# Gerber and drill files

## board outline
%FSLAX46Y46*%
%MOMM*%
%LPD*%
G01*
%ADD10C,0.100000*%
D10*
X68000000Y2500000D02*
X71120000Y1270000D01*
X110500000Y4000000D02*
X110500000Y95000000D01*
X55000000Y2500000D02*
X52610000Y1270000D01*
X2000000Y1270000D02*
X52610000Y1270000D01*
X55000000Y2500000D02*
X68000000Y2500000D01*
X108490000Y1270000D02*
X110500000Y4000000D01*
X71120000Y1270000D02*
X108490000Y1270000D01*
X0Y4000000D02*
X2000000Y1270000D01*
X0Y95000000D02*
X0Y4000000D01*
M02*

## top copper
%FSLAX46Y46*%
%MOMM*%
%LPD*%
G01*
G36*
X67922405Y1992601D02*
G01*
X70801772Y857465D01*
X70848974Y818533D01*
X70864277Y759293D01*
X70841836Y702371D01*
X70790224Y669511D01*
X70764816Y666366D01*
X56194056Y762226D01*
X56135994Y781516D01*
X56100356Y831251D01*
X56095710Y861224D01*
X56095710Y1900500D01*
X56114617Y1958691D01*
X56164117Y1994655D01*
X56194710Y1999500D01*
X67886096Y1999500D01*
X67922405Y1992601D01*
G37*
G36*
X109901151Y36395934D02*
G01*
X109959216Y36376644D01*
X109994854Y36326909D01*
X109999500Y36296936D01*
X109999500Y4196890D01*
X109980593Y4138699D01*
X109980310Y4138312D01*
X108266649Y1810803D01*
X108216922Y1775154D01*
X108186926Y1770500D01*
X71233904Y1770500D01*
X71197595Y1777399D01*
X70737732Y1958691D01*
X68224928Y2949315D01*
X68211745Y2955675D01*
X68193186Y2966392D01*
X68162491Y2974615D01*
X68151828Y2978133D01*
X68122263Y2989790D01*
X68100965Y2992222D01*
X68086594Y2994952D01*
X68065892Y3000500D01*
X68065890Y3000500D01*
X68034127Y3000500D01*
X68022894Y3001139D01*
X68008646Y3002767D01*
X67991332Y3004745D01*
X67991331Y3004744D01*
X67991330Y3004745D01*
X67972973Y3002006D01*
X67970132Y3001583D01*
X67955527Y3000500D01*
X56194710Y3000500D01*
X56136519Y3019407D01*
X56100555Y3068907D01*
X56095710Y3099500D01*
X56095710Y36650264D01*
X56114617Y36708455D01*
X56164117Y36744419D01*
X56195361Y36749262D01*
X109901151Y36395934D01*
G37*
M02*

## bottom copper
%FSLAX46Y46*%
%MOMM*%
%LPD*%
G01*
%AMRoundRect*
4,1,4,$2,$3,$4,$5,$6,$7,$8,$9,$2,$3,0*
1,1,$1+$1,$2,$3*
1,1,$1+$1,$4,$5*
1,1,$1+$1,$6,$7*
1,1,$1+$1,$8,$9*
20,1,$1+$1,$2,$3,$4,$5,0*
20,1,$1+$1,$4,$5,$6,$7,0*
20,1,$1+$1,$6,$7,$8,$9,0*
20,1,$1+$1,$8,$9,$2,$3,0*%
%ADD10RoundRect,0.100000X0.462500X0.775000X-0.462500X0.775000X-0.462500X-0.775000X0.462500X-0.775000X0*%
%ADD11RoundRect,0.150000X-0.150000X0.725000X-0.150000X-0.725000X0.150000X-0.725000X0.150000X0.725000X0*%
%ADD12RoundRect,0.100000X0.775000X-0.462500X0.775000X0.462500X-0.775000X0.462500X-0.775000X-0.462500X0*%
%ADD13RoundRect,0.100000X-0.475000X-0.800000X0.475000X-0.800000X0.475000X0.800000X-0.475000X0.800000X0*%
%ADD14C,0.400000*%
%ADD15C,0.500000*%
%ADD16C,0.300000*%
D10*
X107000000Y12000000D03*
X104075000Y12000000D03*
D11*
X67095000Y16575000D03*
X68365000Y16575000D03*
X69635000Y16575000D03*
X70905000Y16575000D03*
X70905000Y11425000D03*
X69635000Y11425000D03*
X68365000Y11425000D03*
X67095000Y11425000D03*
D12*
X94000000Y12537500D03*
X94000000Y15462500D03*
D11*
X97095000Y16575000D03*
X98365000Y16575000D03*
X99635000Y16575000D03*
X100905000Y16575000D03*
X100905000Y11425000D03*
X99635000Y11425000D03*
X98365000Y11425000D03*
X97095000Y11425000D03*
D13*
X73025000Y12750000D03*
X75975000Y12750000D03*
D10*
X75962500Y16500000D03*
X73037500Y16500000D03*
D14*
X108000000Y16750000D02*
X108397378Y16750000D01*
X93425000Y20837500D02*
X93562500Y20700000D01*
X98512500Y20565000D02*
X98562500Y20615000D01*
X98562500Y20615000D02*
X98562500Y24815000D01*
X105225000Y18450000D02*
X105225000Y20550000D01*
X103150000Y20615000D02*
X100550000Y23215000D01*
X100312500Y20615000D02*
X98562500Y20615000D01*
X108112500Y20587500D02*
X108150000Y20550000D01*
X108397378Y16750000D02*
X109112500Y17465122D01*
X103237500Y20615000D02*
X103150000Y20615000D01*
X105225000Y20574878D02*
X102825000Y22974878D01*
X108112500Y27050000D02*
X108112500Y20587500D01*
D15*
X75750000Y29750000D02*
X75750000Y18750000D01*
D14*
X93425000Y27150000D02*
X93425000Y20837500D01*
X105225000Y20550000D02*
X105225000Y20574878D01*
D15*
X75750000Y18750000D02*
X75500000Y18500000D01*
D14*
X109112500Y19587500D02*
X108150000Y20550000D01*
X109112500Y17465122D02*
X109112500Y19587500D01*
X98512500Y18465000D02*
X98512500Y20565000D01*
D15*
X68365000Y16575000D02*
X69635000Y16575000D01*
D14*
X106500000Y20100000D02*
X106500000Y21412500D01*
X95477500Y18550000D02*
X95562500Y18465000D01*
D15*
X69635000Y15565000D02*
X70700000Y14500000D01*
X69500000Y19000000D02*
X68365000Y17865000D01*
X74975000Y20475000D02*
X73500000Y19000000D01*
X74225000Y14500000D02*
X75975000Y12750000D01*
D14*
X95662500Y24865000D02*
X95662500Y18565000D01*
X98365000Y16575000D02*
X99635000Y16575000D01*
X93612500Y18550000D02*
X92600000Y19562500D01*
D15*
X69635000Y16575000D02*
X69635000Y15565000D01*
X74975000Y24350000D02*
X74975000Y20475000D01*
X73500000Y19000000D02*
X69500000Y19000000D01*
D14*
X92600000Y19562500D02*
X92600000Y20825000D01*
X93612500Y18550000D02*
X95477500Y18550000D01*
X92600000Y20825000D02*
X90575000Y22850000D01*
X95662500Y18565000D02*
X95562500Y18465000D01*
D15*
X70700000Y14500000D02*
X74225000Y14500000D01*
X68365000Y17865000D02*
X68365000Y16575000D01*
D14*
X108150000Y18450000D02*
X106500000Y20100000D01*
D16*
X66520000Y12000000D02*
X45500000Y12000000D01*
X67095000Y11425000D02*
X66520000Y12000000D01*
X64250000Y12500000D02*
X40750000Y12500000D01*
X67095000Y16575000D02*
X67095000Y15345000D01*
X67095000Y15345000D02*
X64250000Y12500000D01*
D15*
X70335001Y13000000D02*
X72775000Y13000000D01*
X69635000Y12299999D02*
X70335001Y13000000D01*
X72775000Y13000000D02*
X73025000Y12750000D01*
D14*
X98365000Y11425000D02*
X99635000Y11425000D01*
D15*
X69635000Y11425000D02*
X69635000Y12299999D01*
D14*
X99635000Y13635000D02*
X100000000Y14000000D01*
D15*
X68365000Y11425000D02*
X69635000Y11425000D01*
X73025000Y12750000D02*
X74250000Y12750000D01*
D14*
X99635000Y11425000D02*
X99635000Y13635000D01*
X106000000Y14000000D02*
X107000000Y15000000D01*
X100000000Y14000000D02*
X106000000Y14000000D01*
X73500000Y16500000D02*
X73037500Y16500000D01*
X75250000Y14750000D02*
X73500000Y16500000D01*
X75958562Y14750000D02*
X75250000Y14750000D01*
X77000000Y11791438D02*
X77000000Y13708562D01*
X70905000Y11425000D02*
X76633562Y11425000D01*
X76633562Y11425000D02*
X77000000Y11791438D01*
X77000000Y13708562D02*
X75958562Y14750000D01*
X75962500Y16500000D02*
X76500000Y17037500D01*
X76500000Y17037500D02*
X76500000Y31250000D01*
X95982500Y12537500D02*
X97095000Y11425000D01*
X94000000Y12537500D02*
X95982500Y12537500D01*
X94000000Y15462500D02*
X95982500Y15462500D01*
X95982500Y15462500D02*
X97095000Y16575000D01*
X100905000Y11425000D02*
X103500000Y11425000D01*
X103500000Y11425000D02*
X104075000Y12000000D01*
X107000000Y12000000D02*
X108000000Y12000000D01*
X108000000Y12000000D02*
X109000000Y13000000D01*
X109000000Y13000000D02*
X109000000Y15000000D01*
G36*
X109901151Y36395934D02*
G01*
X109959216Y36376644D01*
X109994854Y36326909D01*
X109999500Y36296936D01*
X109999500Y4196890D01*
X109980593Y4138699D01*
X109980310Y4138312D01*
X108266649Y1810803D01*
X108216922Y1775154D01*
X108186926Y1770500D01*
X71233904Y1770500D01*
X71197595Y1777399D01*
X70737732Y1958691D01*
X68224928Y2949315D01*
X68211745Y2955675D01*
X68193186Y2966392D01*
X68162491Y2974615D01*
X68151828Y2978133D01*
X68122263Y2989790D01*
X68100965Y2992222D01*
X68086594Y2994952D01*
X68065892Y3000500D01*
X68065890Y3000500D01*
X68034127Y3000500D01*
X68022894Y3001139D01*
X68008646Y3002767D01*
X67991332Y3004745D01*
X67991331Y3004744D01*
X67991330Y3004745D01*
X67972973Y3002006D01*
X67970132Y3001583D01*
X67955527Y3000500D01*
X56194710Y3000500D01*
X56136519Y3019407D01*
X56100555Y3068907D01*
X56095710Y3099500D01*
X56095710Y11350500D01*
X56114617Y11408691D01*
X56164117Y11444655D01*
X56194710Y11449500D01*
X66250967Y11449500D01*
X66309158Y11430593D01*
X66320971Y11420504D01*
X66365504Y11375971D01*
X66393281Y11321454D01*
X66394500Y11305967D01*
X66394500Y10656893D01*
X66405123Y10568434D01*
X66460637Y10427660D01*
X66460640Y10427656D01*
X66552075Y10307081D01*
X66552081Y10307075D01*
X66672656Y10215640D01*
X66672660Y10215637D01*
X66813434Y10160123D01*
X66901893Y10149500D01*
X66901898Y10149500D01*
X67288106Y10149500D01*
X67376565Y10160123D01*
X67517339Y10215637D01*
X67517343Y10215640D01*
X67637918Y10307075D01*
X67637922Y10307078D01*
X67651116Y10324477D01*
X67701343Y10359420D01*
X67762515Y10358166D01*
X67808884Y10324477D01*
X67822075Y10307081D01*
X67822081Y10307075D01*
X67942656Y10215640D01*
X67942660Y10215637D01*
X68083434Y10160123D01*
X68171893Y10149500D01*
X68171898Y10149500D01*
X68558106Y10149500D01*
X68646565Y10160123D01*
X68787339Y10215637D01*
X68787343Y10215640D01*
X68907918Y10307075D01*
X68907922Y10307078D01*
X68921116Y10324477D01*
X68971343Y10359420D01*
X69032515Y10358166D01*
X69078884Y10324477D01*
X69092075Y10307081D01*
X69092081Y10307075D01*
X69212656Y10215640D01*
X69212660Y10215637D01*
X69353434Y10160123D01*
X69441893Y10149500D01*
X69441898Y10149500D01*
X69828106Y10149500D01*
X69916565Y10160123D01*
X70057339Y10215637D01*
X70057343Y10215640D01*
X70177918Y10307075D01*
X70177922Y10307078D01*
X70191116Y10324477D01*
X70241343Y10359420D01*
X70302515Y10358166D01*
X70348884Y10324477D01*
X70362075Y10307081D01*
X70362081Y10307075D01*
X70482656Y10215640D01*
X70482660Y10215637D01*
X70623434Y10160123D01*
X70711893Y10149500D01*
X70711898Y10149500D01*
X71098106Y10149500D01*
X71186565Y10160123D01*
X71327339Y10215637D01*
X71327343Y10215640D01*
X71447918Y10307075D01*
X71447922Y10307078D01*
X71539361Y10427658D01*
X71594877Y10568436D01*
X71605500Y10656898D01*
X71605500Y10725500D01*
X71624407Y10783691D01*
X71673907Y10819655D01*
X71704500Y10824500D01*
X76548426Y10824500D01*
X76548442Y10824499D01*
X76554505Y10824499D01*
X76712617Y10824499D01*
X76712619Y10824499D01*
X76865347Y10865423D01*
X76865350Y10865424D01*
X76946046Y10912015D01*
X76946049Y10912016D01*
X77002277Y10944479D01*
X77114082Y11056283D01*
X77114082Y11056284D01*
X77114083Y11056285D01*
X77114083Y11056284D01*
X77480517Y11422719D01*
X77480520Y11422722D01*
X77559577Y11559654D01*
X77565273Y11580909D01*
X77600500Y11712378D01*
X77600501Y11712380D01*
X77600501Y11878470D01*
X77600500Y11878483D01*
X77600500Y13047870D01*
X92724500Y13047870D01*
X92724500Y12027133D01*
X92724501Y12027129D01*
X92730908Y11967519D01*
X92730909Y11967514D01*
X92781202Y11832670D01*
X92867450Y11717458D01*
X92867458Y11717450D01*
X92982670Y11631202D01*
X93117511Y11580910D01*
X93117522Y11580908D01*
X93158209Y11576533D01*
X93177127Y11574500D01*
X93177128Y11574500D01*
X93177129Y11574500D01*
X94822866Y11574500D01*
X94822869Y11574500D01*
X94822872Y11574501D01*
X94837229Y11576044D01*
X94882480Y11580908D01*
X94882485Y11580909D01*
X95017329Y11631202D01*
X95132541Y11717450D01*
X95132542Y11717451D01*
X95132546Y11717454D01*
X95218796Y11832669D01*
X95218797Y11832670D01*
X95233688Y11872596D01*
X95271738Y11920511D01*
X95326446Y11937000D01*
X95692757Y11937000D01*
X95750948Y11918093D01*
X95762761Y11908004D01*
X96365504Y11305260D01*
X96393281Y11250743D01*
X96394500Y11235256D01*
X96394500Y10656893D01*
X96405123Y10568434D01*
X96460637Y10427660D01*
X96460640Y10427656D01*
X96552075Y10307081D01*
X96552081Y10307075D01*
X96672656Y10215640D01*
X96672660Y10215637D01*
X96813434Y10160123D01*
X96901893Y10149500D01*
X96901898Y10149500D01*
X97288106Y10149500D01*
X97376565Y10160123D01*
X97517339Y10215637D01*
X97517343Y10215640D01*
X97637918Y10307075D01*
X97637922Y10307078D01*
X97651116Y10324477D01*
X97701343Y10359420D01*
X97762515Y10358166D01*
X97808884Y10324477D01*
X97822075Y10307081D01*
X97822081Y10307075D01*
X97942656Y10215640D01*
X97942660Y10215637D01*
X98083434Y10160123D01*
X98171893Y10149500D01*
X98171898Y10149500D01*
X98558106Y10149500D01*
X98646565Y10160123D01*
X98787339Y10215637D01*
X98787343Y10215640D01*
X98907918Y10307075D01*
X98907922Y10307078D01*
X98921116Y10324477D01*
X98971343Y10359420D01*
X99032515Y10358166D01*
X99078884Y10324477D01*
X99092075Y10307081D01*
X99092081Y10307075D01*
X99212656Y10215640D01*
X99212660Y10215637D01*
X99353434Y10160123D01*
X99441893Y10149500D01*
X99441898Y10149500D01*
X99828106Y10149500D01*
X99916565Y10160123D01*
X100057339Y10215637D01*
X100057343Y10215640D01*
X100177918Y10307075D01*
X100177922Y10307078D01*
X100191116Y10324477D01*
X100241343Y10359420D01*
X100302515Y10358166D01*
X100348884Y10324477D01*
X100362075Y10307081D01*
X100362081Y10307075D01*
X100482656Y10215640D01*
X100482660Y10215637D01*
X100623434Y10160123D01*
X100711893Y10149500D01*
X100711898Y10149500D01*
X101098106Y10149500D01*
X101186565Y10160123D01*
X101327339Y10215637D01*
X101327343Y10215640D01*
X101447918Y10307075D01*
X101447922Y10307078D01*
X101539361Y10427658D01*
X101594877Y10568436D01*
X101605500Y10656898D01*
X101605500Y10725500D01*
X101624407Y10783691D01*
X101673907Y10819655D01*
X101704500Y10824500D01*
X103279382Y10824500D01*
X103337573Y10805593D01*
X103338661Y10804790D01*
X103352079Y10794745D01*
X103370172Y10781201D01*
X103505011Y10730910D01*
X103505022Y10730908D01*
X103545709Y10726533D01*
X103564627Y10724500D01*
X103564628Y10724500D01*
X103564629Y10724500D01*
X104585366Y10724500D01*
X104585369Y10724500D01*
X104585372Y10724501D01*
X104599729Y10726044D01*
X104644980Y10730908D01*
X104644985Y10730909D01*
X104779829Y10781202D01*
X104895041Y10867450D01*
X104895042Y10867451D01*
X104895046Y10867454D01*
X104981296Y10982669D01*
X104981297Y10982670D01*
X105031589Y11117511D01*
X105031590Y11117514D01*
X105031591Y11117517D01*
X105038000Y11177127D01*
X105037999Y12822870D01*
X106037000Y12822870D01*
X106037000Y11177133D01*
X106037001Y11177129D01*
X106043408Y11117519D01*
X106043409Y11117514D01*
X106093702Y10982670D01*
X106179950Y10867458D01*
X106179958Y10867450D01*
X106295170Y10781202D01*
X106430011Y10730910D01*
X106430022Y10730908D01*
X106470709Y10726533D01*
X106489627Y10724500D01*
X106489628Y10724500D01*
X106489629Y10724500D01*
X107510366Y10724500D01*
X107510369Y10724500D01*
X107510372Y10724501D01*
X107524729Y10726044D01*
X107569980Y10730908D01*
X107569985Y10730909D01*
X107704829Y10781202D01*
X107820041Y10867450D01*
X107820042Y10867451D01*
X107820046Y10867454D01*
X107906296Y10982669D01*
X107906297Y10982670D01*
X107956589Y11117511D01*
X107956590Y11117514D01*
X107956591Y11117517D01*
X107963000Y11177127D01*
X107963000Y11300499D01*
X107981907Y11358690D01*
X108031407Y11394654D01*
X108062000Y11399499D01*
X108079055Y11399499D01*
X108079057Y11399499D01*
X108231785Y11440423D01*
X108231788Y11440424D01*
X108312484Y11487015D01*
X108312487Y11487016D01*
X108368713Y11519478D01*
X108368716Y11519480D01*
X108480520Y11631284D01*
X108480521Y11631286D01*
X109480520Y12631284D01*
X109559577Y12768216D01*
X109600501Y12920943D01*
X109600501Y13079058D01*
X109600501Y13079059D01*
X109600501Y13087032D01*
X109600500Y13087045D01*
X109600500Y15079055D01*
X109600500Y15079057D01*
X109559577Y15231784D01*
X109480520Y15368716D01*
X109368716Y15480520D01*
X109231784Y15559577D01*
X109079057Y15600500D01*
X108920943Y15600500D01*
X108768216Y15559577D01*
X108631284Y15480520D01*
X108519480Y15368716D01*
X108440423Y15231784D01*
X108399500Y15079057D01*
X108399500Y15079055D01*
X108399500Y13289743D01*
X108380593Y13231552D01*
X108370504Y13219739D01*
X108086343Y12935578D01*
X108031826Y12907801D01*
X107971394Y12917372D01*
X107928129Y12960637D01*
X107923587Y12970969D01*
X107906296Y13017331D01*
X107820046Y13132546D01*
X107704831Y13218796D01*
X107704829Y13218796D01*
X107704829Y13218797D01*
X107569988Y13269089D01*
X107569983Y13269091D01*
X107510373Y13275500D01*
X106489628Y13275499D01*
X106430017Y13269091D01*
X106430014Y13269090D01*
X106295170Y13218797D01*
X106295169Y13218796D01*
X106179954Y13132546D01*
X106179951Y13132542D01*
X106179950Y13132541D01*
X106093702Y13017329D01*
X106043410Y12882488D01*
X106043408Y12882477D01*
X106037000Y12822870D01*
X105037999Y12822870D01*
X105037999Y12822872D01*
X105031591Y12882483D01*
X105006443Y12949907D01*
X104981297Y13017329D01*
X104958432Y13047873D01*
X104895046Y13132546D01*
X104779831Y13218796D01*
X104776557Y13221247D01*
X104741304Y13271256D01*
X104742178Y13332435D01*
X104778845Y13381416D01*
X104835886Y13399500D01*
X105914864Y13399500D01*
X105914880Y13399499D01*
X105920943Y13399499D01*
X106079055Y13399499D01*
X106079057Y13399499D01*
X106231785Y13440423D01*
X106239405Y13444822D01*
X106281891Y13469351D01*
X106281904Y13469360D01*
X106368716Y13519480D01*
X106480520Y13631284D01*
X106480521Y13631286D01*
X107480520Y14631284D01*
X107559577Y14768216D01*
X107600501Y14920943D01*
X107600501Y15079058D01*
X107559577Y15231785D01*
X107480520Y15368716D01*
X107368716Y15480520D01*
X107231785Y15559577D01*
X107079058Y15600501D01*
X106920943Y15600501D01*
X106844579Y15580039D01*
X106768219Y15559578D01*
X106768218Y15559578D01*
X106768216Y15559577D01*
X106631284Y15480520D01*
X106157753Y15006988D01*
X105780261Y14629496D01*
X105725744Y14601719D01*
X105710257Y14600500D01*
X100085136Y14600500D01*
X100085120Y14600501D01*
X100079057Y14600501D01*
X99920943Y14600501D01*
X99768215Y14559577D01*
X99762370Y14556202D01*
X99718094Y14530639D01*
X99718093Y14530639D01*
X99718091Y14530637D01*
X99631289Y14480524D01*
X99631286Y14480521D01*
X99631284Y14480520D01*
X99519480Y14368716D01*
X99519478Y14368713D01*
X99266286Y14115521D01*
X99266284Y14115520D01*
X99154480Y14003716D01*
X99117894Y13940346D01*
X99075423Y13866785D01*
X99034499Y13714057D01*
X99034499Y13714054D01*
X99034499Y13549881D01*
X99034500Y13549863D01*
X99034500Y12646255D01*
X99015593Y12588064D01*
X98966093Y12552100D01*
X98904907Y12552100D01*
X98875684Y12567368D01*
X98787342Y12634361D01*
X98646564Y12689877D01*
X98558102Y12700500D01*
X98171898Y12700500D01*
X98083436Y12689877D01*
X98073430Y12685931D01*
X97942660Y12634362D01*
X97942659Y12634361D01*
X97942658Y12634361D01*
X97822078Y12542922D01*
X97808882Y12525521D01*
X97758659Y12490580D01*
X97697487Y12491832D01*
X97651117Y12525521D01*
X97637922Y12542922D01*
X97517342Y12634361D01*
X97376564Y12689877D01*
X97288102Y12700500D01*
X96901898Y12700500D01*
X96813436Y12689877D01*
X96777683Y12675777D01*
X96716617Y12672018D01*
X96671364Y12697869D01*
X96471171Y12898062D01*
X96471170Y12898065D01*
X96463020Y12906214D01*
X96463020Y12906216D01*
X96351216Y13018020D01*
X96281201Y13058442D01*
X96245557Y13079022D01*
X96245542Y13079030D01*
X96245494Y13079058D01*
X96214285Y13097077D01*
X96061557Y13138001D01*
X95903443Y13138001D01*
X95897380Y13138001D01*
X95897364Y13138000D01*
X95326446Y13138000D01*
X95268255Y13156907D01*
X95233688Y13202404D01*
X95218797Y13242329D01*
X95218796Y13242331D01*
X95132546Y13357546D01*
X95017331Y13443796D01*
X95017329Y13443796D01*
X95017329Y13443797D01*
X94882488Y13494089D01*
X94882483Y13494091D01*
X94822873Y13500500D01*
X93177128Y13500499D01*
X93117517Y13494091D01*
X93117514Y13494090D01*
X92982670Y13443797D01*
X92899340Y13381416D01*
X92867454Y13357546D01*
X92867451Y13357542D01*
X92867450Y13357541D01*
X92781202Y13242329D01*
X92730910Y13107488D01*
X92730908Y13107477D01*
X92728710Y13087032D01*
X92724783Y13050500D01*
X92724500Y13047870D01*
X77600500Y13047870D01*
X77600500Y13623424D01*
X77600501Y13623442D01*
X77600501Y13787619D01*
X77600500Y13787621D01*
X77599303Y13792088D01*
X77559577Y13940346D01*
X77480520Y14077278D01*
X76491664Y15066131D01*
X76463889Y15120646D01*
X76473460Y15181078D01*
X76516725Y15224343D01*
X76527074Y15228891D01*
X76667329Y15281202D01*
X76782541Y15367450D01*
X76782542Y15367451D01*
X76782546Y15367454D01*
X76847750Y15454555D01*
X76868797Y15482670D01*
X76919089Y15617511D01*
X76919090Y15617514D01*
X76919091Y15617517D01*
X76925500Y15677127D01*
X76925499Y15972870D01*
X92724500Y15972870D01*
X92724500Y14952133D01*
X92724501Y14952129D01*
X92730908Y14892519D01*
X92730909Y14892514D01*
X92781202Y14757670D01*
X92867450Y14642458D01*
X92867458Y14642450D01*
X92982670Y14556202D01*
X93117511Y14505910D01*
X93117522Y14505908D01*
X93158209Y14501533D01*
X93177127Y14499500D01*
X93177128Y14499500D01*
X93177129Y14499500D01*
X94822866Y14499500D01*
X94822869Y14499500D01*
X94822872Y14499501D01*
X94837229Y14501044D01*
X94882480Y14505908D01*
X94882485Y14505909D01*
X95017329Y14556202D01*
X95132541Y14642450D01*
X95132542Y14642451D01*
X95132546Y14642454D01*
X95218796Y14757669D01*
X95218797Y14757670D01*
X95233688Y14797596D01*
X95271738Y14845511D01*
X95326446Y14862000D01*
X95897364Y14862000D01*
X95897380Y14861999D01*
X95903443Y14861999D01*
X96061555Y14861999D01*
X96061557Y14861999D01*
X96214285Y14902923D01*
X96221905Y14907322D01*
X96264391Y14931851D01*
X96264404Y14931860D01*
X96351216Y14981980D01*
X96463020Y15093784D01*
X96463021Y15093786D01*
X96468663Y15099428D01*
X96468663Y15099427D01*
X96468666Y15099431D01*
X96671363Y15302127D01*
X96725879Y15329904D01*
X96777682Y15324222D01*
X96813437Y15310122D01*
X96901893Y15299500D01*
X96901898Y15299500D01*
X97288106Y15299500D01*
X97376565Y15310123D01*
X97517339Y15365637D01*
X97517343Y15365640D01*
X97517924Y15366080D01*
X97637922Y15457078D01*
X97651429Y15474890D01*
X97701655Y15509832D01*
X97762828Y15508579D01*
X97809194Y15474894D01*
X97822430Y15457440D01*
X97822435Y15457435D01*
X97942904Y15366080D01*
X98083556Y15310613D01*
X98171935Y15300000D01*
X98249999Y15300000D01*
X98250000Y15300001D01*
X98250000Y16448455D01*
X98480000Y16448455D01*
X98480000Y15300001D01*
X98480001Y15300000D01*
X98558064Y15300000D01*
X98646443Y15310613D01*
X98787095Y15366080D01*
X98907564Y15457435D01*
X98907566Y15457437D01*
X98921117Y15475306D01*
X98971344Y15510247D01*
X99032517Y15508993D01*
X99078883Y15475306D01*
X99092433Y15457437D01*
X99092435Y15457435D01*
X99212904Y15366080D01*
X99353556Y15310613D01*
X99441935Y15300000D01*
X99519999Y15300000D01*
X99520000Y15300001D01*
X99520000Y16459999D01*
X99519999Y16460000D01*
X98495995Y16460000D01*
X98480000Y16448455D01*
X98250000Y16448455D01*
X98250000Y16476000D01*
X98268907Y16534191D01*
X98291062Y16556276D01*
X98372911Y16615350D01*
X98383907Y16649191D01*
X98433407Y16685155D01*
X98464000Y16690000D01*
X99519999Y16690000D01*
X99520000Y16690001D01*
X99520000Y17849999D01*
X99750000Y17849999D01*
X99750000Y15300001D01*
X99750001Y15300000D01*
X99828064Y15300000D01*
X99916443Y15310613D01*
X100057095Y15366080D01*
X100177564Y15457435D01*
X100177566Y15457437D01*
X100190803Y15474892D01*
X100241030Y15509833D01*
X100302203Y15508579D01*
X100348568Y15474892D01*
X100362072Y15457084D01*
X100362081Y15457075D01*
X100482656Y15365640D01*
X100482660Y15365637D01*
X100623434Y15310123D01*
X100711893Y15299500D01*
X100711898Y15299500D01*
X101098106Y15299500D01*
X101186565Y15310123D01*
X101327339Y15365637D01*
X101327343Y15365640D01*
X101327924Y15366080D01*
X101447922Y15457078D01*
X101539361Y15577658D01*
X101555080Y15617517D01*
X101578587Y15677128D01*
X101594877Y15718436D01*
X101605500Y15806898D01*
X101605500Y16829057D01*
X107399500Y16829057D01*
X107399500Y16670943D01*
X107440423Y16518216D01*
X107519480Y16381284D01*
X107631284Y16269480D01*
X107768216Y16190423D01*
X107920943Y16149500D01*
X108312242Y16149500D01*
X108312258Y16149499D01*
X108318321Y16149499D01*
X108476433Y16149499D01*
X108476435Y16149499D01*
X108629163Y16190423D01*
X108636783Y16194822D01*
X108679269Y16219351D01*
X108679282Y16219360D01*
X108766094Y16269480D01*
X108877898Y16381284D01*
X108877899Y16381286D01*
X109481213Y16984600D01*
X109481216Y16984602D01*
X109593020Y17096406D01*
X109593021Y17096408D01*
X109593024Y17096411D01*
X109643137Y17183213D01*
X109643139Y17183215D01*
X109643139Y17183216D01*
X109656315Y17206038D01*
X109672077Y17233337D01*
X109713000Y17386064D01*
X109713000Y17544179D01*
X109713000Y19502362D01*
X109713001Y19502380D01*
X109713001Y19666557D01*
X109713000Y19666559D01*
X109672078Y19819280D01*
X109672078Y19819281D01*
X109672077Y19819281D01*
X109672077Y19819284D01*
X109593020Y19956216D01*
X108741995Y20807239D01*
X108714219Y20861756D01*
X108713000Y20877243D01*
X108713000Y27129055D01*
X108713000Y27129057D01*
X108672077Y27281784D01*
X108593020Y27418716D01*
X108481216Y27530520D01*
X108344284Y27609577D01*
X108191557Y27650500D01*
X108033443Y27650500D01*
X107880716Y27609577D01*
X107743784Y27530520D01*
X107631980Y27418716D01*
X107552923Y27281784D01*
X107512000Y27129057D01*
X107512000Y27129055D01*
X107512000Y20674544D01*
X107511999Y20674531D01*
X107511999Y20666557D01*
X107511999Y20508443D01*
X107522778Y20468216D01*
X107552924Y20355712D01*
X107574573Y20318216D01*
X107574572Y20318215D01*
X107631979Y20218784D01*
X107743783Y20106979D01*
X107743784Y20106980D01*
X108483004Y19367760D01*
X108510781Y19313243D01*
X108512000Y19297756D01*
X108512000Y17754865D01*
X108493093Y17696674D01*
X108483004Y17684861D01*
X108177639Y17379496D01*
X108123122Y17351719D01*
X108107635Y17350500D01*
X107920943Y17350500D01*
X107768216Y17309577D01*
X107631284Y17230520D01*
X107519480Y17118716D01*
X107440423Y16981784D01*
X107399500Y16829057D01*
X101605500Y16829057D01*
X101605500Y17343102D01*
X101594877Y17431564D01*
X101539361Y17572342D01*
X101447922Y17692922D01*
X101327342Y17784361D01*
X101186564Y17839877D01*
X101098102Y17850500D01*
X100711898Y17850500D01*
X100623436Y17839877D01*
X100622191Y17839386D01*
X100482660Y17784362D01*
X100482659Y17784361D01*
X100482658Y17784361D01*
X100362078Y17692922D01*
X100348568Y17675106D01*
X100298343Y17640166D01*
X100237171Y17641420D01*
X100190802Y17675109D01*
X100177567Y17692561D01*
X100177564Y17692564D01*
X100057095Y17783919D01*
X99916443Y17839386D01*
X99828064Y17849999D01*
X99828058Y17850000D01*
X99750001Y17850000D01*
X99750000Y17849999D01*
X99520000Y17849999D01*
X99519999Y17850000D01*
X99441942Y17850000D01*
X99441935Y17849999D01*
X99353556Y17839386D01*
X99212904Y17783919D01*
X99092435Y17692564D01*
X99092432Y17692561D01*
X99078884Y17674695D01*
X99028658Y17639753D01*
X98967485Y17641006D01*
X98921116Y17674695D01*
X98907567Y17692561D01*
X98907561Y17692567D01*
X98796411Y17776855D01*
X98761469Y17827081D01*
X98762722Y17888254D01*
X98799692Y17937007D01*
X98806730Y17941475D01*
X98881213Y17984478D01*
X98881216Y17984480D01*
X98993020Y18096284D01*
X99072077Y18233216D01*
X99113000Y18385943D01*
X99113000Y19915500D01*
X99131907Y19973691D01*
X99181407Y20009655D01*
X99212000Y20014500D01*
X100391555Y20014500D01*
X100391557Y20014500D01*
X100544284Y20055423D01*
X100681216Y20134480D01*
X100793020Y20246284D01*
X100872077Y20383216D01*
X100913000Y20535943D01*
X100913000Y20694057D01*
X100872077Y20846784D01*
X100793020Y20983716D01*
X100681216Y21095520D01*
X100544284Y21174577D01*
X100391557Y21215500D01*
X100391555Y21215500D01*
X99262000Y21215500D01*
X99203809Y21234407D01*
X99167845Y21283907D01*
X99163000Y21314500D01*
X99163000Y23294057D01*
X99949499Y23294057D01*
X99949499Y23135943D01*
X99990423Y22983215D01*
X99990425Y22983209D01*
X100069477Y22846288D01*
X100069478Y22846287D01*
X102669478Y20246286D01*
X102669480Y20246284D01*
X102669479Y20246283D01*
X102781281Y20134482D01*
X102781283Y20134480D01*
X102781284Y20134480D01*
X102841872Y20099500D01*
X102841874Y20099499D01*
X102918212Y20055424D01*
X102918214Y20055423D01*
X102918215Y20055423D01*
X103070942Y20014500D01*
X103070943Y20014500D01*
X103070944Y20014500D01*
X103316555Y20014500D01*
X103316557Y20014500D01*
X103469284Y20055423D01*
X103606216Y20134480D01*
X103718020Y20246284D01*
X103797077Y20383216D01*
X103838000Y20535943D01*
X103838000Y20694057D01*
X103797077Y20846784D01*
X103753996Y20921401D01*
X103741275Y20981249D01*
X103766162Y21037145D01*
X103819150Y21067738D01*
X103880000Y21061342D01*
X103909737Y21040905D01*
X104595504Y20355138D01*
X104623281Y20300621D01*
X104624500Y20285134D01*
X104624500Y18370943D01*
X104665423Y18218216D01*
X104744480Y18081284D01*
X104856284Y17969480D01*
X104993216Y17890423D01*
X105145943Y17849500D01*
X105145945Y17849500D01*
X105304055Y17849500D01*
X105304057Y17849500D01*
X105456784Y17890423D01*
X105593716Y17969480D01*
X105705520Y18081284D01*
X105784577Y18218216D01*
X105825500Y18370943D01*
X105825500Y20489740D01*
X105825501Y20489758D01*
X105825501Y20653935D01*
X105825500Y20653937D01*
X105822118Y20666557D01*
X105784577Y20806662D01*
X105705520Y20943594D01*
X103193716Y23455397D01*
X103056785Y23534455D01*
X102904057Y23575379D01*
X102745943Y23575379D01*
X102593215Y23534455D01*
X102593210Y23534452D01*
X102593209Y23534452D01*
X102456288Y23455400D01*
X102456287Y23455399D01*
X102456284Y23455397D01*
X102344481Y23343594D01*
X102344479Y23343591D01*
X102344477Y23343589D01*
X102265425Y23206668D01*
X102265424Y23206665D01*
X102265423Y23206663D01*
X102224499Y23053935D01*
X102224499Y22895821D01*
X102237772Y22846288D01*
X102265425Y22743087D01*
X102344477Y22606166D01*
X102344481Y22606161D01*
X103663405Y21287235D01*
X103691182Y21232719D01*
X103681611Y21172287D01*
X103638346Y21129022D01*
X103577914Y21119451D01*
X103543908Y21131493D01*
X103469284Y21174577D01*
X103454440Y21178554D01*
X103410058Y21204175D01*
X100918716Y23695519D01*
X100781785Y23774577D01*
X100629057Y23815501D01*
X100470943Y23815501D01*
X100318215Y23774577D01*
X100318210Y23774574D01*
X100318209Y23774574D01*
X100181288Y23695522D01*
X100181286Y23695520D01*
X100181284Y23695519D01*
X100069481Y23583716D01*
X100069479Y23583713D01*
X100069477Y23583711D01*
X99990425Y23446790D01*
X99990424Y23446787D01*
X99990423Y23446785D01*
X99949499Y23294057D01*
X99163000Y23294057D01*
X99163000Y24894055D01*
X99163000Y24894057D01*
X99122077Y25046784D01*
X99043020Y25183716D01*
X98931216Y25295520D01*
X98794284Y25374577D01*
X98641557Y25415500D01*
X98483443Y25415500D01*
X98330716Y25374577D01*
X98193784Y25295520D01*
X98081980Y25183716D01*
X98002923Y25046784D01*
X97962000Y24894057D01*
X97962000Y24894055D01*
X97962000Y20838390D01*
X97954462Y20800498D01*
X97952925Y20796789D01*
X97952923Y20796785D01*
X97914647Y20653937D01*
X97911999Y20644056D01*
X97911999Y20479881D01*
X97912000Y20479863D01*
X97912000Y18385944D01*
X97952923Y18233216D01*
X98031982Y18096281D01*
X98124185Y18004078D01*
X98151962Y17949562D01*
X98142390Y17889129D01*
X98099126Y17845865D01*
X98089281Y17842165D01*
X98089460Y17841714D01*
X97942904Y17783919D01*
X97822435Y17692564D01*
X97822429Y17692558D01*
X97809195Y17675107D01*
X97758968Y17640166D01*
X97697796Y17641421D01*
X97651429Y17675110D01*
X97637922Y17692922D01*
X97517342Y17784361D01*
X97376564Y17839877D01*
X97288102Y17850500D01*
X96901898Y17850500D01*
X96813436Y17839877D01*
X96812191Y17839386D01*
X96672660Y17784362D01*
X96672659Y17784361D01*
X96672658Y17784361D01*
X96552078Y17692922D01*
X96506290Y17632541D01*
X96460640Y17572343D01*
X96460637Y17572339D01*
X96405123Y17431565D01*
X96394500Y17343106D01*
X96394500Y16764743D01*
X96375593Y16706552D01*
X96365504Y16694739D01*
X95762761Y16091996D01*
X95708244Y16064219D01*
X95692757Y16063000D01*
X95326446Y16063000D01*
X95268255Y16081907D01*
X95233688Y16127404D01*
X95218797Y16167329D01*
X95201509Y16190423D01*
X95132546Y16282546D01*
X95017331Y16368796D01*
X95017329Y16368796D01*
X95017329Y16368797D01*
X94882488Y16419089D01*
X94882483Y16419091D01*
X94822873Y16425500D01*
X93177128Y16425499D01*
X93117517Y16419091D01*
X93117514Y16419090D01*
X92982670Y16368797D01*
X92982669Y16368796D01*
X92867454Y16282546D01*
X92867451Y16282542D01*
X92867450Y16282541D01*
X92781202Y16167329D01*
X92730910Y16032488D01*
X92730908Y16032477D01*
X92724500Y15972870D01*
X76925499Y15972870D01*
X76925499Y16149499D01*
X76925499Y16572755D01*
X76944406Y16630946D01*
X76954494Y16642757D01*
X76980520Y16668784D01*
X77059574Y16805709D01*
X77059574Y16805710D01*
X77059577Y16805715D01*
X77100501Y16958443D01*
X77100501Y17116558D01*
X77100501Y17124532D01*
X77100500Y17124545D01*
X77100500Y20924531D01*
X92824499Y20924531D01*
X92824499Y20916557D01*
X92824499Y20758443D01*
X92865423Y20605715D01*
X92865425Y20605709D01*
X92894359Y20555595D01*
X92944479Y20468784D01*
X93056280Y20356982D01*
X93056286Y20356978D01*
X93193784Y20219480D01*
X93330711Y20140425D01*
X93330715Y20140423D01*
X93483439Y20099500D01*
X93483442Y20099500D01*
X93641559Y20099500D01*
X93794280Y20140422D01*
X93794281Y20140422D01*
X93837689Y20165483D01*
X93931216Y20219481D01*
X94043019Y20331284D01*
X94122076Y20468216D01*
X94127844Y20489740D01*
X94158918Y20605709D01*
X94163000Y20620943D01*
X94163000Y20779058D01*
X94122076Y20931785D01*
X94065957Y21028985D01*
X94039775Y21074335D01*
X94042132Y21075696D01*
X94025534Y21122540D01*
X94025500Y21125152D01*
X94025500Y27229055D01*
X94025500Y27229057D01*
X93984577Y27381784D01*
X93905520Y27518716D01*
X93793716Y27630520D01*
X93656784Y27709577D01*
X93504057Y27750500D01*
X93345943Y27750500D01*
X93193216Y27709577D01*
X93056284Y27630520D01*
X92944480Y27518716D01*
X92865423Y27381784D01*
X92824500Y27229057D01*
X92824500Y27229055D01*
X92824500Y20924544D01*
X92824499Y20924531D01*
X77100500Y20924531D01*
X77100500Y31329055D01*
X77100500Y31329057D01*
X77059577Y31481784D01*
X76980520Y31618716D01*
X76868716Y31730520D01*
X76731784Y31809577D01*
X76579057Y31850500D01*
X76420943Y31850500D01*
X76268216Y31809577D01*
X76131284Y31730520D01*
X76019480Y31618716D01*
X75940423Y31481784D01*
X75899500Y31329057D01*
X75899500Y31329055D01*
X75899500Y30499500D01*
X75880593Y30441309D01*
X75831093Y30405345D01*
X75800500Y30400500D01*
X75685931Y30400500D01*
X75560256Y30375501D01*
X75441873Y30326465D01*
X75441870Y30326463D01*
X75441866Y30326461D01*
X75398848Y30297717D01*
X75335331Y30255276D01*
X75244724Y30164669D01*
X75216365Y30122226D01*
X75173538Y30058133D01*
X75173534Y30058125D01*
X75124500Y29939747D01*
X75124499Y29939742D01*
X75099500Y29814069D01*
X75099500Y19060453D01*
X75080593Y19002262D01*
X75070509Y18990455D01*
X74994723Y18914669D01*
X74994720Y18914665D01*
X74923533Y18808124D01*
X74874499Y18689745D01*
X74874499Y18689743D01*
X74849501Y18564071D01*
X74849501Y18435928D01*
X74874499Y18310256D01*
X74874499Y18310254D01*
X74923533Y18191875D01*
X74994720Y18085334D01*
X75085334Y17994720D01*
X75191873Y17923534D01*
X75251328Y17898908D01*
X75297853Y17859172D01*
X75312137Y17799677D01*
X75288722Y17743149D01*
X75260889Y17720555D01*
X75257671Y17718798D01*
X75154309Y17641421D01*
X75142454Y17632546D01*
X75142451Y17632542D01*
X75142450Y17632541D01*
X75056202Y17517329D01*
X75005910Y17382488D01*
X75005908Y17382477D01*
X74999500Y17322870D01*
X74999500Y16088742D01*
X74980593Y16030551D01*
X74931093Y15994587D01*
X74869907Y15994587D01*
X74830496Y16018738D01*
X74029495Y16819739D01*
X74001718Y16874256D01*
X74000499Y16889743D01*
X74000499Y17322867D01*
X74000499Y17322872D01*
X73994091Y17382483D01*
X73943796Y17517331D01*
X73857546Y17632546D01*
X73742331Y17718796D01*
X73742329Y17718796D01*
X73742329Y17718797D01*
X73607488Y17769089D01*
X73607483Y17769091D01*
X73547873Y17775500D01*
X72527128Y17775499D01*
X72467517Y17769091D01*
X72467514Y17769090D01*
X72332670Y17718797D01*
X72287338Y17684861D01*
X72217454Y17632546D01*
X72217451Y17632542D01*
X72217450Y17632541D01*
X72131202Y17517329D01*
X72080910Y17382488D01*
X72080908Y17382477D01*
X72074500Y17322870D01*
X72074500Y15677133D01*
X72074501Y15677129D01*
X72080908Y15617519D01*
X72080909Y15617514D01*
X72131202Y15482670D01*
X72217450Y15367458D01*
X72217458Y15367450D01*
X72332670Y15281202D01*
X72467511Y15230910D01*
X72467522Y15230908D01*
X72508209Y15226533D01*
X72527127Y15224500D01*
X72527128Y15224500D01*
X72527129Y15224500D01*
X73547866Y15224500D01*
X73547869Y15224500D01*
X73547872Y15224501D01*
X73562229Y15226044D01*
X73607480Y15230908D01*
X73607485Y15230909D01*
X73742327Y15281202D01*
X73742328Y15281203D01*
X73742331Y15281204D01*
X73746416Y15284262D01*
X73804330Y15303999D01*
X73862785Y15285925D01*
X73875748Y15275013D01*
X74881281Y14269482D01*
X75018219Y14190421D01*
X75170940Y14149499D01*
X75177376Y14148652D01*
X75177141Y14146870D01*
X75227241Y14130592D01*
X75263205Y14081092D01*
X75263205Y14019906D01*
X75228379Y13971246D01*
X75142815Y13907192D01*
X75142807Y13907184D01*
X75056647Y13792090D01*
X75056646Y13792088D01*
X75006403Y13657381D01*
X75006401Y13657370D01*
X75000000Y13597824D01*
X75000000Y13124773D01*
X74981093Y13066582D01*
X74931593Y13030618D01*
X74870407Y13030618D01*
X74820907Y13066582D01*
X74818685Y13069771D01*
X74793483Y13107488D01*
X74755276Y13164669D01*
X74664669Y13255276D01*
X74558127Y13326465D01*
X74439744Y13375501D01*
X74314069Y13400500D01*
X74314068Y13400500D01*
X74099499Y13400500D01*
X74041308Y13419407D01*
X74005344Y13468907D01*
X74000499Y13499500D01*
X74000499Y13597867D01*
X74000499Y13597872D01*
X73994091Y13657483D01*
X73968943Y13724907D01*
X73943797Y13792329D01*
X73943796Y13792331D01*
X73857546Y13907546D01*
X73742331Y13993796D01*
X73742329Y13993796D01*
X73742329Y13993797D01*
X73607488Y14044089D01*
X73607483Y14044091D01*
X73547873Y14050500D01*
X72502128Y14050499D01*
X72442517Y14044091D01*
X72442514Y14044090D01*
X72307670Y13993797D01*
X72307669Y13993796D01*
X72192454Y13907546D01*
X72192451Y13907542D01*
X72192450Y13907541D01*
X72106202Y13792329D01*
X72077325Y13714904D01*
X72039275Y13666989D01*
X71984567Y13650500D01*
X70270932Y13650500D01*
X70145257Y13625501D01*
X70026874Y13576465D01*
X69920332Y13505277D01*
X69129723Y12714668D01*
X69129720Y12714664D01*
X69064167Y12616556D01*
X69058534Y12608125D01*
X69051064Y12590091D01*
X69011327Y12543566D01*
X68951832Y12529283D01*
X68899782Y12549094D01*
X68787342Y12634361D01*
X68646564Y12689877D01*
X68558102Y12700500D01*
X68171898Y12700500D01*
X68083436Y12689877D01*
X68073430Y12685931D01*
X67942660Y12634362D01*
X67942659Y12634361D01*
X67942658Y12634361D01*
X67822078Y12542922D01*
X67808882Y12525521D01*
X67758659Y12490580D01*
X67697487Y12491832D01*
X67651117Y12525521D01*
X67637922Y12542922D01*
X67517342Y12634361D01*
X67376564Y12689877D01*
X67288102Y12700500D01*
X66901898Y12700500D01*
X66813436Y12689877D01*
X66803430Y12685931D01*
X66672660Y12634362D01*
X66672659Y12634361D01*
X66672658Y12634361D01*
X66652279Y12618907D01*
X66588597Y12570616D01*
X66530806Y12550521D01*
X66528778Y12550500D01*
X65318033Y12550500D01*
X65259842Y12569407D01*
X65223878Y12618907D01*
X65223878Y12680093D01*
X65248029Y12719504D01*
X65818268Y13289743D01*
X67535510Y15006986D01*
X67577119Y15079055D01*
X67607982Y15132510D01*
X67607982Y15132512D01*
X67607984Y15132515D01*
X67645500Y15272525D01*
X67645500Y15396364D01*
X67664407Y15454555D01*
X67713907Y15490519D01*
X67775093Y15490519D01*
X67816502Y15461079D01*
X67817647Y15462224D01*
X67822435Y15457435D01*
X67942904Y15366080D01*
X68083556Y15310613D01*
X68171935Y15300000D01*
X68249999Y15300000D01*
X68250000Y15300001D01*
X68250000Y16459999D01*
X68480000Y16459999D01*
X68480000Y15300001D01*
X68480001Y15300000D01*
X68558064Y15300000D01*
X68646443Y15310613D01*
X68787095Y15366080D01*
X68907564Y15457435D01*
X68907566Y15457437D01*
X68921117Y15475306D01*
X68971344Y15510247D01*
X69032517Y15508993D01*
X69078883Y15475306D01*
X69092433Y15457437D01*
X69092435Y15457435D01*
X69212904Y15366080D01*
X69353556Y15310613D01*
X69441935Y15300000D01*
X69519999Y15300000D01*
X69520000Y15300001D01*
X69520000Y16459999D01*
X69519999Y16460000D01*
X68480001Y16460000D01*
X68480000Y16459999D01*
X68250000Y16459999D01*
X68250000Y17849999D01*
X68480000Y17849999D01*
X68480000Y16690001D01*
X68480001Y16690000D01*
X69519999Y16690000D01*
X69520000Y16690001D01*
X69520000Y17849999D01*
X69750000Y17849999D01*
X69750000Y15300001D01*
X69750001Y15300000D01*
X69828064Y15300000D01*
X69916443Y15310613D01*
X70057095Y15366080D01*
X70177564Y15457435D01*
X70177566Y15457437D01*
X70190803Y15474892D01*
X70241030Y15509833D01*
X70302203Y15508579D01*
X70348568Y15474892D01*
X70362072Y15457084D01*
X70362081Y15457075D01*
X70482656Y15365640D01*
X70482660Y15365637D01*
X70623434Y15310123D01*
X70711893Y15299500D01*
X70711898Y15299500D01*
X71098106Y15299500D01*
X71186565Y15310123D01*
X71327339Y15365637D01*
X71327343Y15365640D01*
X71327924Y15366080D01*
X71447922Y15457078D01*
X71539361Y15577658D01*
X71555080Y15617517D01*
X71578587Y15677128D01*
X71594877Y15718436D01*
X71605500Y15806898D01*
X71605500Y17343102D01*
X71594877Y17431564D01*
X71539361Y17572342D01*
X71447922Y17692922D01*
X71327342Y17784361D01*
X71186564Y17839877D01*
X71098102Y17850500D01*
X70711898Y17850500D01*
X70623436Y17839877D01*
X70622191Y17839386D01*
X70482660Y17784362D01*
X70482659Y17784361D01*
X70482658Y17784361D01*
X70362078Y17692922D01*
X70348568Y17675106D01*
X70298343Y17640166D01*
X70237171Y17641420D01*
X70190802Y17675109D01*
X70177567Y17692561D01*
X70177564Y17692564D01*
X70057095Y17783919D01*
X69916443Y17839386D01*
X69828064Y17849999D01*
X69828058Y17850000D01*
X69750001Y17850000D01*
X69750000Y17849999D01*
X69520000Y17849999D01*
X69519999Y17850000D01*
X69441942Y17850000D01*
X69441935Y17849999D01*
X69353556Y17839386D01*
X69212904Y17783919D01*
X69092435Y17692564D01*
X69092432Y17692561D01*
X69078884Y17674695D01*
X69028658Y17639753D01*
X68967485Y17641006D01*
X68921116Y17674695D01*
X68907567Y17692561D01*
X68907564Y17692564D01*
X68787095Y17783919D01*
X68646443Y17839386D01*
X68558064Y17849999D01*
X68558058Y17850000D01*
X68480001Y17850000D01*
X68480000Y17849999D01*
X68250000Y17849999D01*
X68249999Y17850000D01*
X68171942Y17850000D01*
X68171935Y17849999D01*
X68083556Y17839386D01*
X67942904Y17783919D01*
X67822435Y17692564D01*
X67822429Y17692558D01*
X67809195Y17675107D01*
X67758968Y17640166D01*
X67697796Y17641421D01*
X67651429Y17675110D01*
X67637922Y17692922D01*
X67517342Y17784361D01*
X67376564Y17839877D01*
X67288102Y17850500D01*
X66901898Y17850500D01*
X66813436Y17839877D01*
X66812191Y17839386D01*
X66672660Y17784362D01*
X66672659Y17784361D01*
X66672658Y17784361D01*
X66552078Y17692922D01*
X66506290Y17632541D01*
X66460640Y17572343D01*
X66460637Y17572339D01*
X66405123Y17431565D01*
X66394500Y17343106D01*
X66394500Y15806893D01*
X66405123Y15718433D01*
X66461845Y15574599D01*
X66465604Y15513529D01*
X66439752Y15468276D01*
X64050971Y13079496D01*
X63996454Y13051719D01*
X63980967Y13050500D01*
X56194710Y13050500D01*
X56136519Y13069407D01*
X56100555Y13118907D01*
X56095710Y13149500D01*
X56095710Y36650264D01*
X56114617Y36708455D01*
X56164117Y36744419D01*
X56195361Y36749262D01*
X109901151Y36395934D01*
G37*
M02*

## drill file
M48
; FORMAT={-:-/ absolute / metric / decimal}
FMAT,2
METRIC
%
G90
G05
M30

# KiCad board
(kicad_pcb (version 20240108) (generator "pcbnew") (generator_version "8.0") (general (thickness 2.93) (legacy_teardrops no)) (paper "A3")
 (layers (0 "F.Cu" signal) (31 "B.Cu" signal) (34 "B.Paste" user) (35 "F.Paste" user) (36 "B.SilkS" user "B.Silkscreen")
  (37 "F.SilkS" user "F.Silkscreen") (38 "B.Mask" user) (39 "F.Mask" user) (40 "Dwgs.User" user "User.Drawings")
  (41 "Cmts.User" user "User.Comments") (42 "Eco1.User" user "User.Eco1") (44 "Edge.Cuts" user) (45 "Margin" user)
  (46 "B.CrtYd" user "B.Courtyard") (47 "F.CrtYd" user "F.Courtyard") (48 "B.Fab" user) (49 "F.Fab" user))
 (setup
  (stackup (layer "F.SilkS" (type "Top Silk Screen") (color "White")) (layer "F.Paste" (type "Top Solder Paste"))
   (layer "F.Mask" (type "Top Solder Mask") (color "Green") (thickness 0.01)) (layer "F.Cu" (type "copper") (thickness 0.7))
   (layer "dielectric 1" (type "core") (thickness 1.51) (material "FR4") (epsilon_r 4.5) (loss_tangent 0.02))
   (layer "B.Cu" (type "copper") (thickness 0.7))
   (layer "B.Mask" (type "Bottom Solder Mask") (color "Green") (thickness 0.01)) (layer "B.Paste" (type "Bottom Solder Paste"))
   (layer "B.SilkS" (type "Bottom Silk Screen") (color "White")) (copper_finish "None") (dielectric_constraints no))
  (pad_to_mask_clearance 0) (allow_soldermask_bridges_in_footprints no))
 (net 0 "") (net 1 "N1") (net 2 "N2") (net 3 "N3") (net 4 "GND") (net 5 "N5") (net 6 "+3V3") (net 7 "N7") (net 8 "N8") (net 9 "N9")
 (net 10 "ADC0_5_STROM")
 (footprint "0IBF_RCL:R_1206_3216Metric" (layer "B.Cu") (at 105.5375 -12 180)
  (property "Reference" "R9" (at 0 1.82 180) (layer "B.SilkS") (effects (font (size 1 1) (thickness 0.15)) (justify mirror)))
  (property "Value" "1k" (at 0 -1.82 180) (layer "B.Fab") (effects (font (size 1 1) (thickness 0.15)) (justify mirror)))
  (pad "1" smd roundrect (at -1.4625 0 180) (size 1.125 1.75) (layers "B.Cu" "B.Paste" "B.Mask") (roundrect_rratio 0.08888888889)
   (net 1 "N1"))
  (pad "2" smd roundrect (at 1.4625 0 180) (size 1.125 1.75) (layers "B.Cu" "B.Paste" "B.Mask") (roundrect_rratio 0.08888888889)
   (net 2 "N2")))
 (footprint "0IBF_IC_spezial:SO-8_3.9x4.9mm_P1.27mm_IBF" (layer "B.Cu") (at 69 -14 -90)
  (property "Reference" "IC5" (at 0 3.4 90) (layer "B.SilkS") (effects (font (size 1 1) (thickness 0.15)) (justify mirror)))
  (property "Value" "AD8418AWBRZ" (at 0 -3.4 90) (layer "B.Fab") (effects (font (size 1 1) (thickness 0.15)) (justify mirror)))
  (pad "1" smd roundrect (at -2.575 1.905 270) (size 1.75 0.6) (layers "B.Cu" "B.Paste" "B.Mask") (roundrect_rratio 0.25) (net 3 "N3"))
  (pad "2" smd roundrect (at -2.575 0.635 270) (size 1.75 0.6) (layers "B.Cu" "B.Paste" "B.Mask") (roundrect_rratio 0.25) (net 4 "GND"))
  (pad "3" smd roundrect (at -2.575 -0.635 270) (size 1.75 0.6) (layers "B.Cu" "B.Paste" "B.Mask") (roundrect_rratio 0.25) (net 4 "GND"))
  (pad "4" smd roundrect (at -2.575 -1.905 270) (size 1.75 0.6) (layers "B.Cu" "B.Paste" "B.Mask") (roundrect_rratio 0.25))
  (pad "5" smd roundrect (at 2.575 -1.905 270) (size 1.75 0.6) (layers "B.Cu" "B.Paste" "B.Mask") (roundrect_rratio 0.25) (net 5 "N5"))
  (pad "6" smd roundrect (at 2.575 -0.635 270) (size 1.75 0.6) (layers "B.Cu" "B.Paste" "B.Mask") (roundrect_rratio 0.25) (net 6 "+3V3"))
  (pad "7" smd roundrect (at 2.575 0.635 270) (size 1.75 0.6) (layers "B.Cu" "B.Paste" "B.Mask") (roundrect_rratio 0.25) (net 6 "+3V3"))
  (pad "8" smd roundrect (at 2.575 1.905 270) (size 1.75 0.6) (layers "B.Cu" "B.Paste" "B.Mask") (roundrect_rratio 0.25) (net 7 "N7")))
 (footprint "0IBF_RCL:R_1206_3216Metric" (layer "B.Cu") (at 94 -14 90)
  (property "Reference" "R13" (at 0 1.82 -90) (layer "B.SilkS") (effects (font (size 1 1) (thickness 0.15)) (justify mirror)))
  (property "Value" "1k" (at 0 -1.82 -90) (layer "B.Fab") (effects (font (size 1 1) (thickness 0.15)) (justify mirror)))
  (pad "1" smd roundrect (at -1.4625 0 90) (size 1.125 1.75) (layers "B.Cu" "B.Paste" "B.Mask") (roundrect_rratio 0.08888888889)
   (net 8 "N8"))
  (pad "2" smd roundrect (at 1.4625 0 90) (size 1.125 1.75) (layers "B.Cu" "B.Paste" "B.Mask") (roundrect_rratio 0.08888888889) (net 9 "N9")))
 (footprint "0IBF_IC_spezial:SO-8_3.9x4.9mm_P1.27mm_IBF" (layer "B.Cu") (at 99 -14 -90)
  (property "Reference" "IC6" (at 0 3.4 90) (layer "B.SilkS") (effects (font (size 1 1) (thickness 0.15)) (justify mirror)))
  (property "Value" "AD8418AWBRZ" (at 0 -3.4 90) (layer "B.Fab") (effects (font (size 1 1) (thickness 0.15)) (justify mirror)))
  (pad "1" smd roundrect (at -2.575 1.905 270) (size 1.75 0.6) (layers "B.Cu" "B.Paste" "B.Mask") (roundrect_rratio 0.25) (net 9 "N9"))
  (pad "2" smd roundrect (at -2.575 0.635 270) (size 1.75 0.6) (layers "B.Cu" "B.Paste" "B.Mask") (roundrect_rratio 0.25) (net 4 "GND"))
  (pad "3" smd roundrect (at -2.575 -0.635 270) (size 1.75 0.6) (layers "B.Cu" "B.Paste" "B.Mask") (roundrect_rratio 0.25) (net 4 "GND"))
  (pad "4" smd roundrect (at -2.575 -1.905 270) (size 1.75 0.6) (layers "B.Cu" "B.Paste" "B.Mask") (roundrect_rratio 0.25))
  (pad "5" smd roundrect (at 2.575 -1.905 270) (size 1.75 0.6) (layers "B.Cu" "B.Paste" "B.Mask") (roundrect_rratio 0.25) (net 2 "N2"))
  (pad "6" smd roundrect (at 2.575 -0.635 270) (size 1.75 0.6) (layers "B.Cu" "B.Paste" "B.Mask") (roundrect_rratio 0.25) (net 6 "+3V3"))
  (pad "7" smd roundrect (at 2.575 0.635 270) (size 1.75 0.6) (layers "B.Cu" "B.Paste" "B.Mask") (roundrect_rratio 0.25) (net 6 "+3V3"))
  (pad "8" smd roundrect (at 2.575 1.905 270) (size 1.75 0.6) (layers "B.Cu" "B.Paste" "B.Mask") (roundrect_rratio 0.25) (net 8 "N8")))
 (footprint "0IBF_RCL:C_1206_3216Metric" (layer "B.Cu") (at 74.5 -12.75)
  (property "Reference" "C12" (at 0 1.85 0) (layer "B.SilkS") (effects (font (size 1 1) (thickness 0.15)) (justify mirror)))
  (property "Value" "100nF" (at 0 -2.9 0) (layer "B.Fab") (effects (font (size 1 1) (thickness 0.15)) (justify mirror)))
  (pad "1" smd roundrect (at -1.475 0) (size 1.15 1.8) (layers "B.Cu" "B.Paste" "B.Mask") (roundrect_rratio 0.08695652174) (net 6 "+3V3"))
  (pad "2" smd roundrect (at 1.475 0) (size 1.15 1.8) (layers "B.Cu" "B.Paste" "B.Mask") (roundrect_rratio 0.08695652174) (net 4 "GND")))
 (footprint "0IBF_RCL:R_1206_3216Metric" (layer "B.Cu") (at 74.5 -16.5 180)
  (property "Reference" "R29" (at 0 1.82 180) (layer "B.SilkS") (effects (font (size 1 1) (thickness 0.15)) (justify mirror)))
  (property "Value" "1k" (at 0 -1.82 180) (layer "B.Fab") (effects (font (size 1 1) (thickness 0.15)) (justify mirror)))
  (pad "1" smd roundrect (at -1.4625 0 180) (size 1.125 1.75) (layers "B.Cu" "B.Paste" "B.Mask") (roundrect_rratio 0.08888888889)
   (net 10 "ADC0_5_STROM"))
  (pad "2" smd roundrect (at 1.4625 0 180) (size 1.125 1.75) (layers "B.Cu" "B.Paste" "B.Mask") (roundrect_rratio 0.08888888889)
   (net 5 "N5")))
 (gr_line (start 68 -2.5) (end 71.12 -1.27) (stroke (width 0.1) (type default)) (layer "Edge.Cuts"))
 (gr_line (start 110.5 -4) (end 110.5 -95) (stroke (width 0.1) (type default)) (layer "Edge.Cuts"))
 (gr_line (start 55 -2.5) (end 52.61 -1.27) (stroke (width 0.1) (type default)) (layer "Edge.Cuts"))
 (gr_line (start 2 -1.27) (end 52.61 -1.27) (stroke (width 0.1) (type default)) (layer "Edge.Cuts"))
 (gr_line (start 55 -2.5) (end 68 -2.5) (stroke (width 0.1) (type default)) (layer "Edge.Cuts"))
 (gr_line (start 108.49 -1.27) (end 110.5 -4) (stroke (width 0.1) (type default)) (layer "Edge.Cuts"))
 (gr_line (start 71.12 -1.27) (end 108.49 -1.27) (stroke (width 0.1) (type default)) (layer "Edge.Cuts"))
 (gr_line (start 0 -4) (end 2 -1.27) (stroke (width 0.1) (type default)) (layer "Edge.Cuts"))
 (gr_line (start 0 -95) (end 0 -4) (stroke (width 0.1) (type default)) (layer "Edge.Cuts"))
 (segment (start 108 -16.75) (end 108.397378 -16.75) (width 0.4) (layer "B.Cu") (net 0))
 (segment (start 93.425 -20.8375) (end 93.5625 -20.7) (width 0.4) (layer "B.Cu") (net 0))
 (segment (start 98.5125 -20.565) (end 98.5625 -20.615) (width 0.4) (layer "B.Cu") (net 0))
 (segment (start 98.5625 -20.615) (end 98.5625 -24.815) (width 0.4) (layer "B.Cu") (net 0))
 (segment (start 105.225 -18.45) (end 105.225 -20.55) (width 0.4) (layer "B.Cu") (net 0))
 (segment (start 103.15 -20.615) (end 100.55 -23.215) (width 0.4) (layer "B.Cu") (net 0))
 (segment (start 100.3125 -20.615) (end 98.5625 -20.615) (width 0.4) (layer "B.Cu") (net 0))
 (segment (start 108.1125 -20.5875) (end 108.15 -20.55) (width 0.4) (layer "B.Cu") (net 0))
 (segment (start 108.397378 -16.75) (end 109.1125 -17.465122) (width 0.4) (layer "B.Cu") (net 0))
 (segment (start 103.2375 -20.615) (end 103.15 -20.615) (width 0.4) (layer "B.Cu") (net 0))
 (segment (start 105.225 -20.574878) (end 102.825 -22.974878) (width 0.4) (layer "B.Cu") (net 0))
 (segment (start 108.1125 -27.05) (end 108.1125 -20.5875) (width 0.4) (layer "B.Cu") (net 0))
 (segment (start 75.75 -29.75) (end 75.75 -18.75) (width 0.5) (layer "B.Cu") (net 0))
 (segment (start 93.425 -27.15) (end 93.425 -20.8375) (width 0.4) (layer "B.Cu") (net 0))
 (segment (start 105.225 -20.55) (end 105.225 -20.574878) (width 0.4) (layer "B.Cu") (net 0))
 (segment (start 75.75 -18.75) (end 75.5 -18.5) (width 0.5) (layer "B.Cu") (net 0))
 (segment (start 109.1125 -19.5875) (end 108.15 -20.55) (width 0.4) (layer "B.Cu") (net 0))
 (segment (start 109.1125 -17.465122) (end 109.1125 -19.5875) (width 0.4) (layer "B.Cu") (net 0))
 (segment (start 98.5125 -18.465) (end 98.5125 -20.565) (width 0.4) (layer "B.Cu") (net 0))
 (segment (start 68.365 -16.575) (end 69.635 -16.575) (width 0.5) (layer "B.Cu") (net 4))
 (segment (start 106.5 -20.1) (end 106.5 -21.4125) (width 0.4) (layer "B.Cu") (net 4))
 (segment (start 95.4775 -18.55) (end 95.5625 -18.465) (width 0.4) (layer "B.Cu") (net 4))
 (segment (start 69.635 -15.565) (end 70.7 -14.5) (width 0.5) (layer "B.Cu") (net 4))
 (segment (start 69.5 -19) (end 68.365 -17.865) (width 0.5) (layer "B.Cu") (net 4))
 (segment (start 74.975 -20.475) (end 73.5 -19) (width 0.5) (layer "B.Cu") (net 4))
 (segment (start 74.225 -14.5) (end 75.975 -12.75) (width 0.5) (layer "B.Cu") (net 4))
 (segment (start 95.6625 -24.865) (end 95.6625 -18.565) (width 0.4) (layer "B.Cu") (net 4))
 (segment (start 98.365 -16.575) (end 99.635 -16.575) (width 0.4) (layer "B.Cu") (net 4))
 (segment (start 93.6125 -18.55) (end 92.6 -19.5625) (width 0.4) (layer "B.Cu") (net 4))
 (segment (start 69.635 -16.575) (end 69.635 -15.565) (width 0.5) (layer "B.Cu") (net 4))
 (segment (start 74.975 -24.35) (end 74.975 -20.475) (width 0.5) (layer "B.Cu") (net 4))
 (segment (start 73.5 -19) (end 69.5 -19) (width 0.5) (layer "B.Cu") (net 4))
 (segment (start 92.6 -19.5625) (end 92.6 -20.825) (width 0.4) (layer "B.Cu") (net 4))
 (segment (start 93.6125 -18.55) (end 95.4775 -18.55) (width 0.4) (layer "B.Cu") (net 4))
 (segment (start 92.6 -20.825) (end 90.575 -22.85) (width 0.4) (layer "B.Cu") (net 4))
 (segment (start 95.6625 -18.565) (end 95.5625 -18.465) (width 0.4) (layer "B.Cu") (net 4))
 (segment (start 70.7 -14.5) (end 74.225 -14.5) (width 0.5) (layer "B.Cu") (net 4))
 (segment (start 68.365 -17.865) (end 68.365 -16.575) (width 0.5) (layer "B.Cu") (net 4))
 (segment (start 108.15 -18.45) (end 106.5 -20.1) (width 0.4) (layer "B.Cu") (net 4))
 (segment (start 66.52 -12) (end 45.5 -12) (width 0.3) (layer "B.Cu") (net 7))
 (segment (start 67.095 -11.425) (end 66.52 -12) (width 0.3) (layer "B.Cu") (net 7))
 (segment (start 64.25 -12.5) (end 40.75 -12.5) (width 0.3) (layer "B.Cu") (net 3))
 (segment (start 67.095 -16.575) (end 67.095 -15.345) (width 0.3) (layer "B.Cu") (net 3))
 (segment (start 67.095 -15.345) (end 64.25 -12.5) (width 0.3) (layer "B.Cu") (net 3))
 (segment (start 70.335001 -13) (end 72.775 -13) (width 0.5) (layer "B.Cu") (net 6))
 (segment (start 69.635 -12.299999) (end 70.335001 -13) (width 0.5) (layer "B.Cu") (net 6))
 (segment (start 72.775 -13) (end 73.025 -12.75) (width 0.5) (layer "B.Cu") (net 6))
 (segment (start 98.365 -11.425) (end 99.635 -11.425) (width 0.4) (layer "B.Cu") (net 6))
 (segment (start 69.635 -11.425) (end 69.635 -12.299999) (width 0.5) (layer "B.Cu") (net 6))
 (segment (start 99.635 -13.635) (end 100 -14) (width 0.4) (layer "B.Cu") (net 6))
 (segment (start 68.365 -11.425) (end 69.635 -11.425) (width 0.5) (layer "B.Cu") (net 6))
 (segment (start 73.025 -12.75) (end 74.25 -12.75) (width 0.5) (layer "B.Cu") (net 6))
 (segment (start 99.635 -11.425) (end 99.635 -13.635) (width 0.4) (layer "B.Cu") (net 6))
 (segment (start 106 -14) (end 107 -15) (width 0.4) (layer "B.Cu") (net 6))
 (segment (start 100 -14) (end 106 -14) (width 0.4) (layer "B.Cu") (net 6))
 (segment (start 73.5 -16.5) (end 73.0375 -16.5) (width 0.4) (layer "B.Cu") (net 5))
 (segment (start 75.25 -14.75) (end 73.5 -16.5) (width 0.4) (layer "B.Cu") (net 5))
 (segment (start 75.958562 -14.75) (end 75.25 -14.75) (width 0.4) (layer "B.Cu") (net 5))
 (segment (start 77 -11.791438) (end 77 -13.708562) (width 0.4) (layer "B.Cu") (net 5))
 (segment (start 70.905 -11.425) (end 76.633562 -11.425) (width 0.4) (layer "B.Cu") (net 5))
 (segment (start 76.633562 -11.425) (end 77 -11.791438) (width 0.4) (layer "B.Cu") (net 5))
 (segment (start 77 -13.708562) (end 75.958562 -14.75) (width 0.4) (layer "B.Cu") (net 5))
 (segment (start 75.9625 -16.5) (end 76.5 -17.0375) (width 0.4) (layer "B.Cu") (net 10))
 (segment (start 76.5 -17.0375) (end 76.5 -31.25) (width 0.4) (layer "B.Cu") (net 10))
 (segment (start 95.9825 -12.5375) (end 97.095 -11.425) (width 0.4) (layer "B.Cu") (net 8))
 (segment (start 94 -12.5375) (end 95.9825 -12.5375) (width 0.4) (layer "B.Cu") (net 8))
 (segment (start 94 -15.4625) (end 95.9825 -15.4625) (width 0.4) (layer "B.Cu") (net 9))
 (segment (start 95.9825 -15.4625) (end 97.095 -16.575) (width 0.4) (layer "B.Cu") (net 9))
 (segment (start 100.905 -11.425) (end 103.5 -11.425) (width 0.4) (layer "B.Cu") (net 2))
 (segment (start 103.5 -11.425) (end 104.075 -12) (width 0.4) (layer "B.Cu") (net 2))
 (segment (start 107 -12) (end 108 -12) (width 0.4) (layer "B.Cu") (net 1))
 (segment (start 108 -12) (end 109 -13) (width 0.4) (layer "B.Cu") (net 1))
 (segment (start 109 -13) (end 109 -15) (width 0.4) (layer "B.Cu") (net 1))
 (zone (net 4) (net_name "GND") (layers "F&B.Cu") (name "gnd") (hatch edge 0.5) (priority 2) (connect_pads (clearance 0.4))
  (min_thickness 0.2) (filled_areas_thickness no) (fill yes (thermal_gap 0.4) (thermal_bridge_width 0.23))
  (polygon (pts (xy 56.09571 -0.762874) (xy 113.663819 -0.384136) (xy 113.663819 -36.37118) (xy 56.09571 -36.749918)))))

